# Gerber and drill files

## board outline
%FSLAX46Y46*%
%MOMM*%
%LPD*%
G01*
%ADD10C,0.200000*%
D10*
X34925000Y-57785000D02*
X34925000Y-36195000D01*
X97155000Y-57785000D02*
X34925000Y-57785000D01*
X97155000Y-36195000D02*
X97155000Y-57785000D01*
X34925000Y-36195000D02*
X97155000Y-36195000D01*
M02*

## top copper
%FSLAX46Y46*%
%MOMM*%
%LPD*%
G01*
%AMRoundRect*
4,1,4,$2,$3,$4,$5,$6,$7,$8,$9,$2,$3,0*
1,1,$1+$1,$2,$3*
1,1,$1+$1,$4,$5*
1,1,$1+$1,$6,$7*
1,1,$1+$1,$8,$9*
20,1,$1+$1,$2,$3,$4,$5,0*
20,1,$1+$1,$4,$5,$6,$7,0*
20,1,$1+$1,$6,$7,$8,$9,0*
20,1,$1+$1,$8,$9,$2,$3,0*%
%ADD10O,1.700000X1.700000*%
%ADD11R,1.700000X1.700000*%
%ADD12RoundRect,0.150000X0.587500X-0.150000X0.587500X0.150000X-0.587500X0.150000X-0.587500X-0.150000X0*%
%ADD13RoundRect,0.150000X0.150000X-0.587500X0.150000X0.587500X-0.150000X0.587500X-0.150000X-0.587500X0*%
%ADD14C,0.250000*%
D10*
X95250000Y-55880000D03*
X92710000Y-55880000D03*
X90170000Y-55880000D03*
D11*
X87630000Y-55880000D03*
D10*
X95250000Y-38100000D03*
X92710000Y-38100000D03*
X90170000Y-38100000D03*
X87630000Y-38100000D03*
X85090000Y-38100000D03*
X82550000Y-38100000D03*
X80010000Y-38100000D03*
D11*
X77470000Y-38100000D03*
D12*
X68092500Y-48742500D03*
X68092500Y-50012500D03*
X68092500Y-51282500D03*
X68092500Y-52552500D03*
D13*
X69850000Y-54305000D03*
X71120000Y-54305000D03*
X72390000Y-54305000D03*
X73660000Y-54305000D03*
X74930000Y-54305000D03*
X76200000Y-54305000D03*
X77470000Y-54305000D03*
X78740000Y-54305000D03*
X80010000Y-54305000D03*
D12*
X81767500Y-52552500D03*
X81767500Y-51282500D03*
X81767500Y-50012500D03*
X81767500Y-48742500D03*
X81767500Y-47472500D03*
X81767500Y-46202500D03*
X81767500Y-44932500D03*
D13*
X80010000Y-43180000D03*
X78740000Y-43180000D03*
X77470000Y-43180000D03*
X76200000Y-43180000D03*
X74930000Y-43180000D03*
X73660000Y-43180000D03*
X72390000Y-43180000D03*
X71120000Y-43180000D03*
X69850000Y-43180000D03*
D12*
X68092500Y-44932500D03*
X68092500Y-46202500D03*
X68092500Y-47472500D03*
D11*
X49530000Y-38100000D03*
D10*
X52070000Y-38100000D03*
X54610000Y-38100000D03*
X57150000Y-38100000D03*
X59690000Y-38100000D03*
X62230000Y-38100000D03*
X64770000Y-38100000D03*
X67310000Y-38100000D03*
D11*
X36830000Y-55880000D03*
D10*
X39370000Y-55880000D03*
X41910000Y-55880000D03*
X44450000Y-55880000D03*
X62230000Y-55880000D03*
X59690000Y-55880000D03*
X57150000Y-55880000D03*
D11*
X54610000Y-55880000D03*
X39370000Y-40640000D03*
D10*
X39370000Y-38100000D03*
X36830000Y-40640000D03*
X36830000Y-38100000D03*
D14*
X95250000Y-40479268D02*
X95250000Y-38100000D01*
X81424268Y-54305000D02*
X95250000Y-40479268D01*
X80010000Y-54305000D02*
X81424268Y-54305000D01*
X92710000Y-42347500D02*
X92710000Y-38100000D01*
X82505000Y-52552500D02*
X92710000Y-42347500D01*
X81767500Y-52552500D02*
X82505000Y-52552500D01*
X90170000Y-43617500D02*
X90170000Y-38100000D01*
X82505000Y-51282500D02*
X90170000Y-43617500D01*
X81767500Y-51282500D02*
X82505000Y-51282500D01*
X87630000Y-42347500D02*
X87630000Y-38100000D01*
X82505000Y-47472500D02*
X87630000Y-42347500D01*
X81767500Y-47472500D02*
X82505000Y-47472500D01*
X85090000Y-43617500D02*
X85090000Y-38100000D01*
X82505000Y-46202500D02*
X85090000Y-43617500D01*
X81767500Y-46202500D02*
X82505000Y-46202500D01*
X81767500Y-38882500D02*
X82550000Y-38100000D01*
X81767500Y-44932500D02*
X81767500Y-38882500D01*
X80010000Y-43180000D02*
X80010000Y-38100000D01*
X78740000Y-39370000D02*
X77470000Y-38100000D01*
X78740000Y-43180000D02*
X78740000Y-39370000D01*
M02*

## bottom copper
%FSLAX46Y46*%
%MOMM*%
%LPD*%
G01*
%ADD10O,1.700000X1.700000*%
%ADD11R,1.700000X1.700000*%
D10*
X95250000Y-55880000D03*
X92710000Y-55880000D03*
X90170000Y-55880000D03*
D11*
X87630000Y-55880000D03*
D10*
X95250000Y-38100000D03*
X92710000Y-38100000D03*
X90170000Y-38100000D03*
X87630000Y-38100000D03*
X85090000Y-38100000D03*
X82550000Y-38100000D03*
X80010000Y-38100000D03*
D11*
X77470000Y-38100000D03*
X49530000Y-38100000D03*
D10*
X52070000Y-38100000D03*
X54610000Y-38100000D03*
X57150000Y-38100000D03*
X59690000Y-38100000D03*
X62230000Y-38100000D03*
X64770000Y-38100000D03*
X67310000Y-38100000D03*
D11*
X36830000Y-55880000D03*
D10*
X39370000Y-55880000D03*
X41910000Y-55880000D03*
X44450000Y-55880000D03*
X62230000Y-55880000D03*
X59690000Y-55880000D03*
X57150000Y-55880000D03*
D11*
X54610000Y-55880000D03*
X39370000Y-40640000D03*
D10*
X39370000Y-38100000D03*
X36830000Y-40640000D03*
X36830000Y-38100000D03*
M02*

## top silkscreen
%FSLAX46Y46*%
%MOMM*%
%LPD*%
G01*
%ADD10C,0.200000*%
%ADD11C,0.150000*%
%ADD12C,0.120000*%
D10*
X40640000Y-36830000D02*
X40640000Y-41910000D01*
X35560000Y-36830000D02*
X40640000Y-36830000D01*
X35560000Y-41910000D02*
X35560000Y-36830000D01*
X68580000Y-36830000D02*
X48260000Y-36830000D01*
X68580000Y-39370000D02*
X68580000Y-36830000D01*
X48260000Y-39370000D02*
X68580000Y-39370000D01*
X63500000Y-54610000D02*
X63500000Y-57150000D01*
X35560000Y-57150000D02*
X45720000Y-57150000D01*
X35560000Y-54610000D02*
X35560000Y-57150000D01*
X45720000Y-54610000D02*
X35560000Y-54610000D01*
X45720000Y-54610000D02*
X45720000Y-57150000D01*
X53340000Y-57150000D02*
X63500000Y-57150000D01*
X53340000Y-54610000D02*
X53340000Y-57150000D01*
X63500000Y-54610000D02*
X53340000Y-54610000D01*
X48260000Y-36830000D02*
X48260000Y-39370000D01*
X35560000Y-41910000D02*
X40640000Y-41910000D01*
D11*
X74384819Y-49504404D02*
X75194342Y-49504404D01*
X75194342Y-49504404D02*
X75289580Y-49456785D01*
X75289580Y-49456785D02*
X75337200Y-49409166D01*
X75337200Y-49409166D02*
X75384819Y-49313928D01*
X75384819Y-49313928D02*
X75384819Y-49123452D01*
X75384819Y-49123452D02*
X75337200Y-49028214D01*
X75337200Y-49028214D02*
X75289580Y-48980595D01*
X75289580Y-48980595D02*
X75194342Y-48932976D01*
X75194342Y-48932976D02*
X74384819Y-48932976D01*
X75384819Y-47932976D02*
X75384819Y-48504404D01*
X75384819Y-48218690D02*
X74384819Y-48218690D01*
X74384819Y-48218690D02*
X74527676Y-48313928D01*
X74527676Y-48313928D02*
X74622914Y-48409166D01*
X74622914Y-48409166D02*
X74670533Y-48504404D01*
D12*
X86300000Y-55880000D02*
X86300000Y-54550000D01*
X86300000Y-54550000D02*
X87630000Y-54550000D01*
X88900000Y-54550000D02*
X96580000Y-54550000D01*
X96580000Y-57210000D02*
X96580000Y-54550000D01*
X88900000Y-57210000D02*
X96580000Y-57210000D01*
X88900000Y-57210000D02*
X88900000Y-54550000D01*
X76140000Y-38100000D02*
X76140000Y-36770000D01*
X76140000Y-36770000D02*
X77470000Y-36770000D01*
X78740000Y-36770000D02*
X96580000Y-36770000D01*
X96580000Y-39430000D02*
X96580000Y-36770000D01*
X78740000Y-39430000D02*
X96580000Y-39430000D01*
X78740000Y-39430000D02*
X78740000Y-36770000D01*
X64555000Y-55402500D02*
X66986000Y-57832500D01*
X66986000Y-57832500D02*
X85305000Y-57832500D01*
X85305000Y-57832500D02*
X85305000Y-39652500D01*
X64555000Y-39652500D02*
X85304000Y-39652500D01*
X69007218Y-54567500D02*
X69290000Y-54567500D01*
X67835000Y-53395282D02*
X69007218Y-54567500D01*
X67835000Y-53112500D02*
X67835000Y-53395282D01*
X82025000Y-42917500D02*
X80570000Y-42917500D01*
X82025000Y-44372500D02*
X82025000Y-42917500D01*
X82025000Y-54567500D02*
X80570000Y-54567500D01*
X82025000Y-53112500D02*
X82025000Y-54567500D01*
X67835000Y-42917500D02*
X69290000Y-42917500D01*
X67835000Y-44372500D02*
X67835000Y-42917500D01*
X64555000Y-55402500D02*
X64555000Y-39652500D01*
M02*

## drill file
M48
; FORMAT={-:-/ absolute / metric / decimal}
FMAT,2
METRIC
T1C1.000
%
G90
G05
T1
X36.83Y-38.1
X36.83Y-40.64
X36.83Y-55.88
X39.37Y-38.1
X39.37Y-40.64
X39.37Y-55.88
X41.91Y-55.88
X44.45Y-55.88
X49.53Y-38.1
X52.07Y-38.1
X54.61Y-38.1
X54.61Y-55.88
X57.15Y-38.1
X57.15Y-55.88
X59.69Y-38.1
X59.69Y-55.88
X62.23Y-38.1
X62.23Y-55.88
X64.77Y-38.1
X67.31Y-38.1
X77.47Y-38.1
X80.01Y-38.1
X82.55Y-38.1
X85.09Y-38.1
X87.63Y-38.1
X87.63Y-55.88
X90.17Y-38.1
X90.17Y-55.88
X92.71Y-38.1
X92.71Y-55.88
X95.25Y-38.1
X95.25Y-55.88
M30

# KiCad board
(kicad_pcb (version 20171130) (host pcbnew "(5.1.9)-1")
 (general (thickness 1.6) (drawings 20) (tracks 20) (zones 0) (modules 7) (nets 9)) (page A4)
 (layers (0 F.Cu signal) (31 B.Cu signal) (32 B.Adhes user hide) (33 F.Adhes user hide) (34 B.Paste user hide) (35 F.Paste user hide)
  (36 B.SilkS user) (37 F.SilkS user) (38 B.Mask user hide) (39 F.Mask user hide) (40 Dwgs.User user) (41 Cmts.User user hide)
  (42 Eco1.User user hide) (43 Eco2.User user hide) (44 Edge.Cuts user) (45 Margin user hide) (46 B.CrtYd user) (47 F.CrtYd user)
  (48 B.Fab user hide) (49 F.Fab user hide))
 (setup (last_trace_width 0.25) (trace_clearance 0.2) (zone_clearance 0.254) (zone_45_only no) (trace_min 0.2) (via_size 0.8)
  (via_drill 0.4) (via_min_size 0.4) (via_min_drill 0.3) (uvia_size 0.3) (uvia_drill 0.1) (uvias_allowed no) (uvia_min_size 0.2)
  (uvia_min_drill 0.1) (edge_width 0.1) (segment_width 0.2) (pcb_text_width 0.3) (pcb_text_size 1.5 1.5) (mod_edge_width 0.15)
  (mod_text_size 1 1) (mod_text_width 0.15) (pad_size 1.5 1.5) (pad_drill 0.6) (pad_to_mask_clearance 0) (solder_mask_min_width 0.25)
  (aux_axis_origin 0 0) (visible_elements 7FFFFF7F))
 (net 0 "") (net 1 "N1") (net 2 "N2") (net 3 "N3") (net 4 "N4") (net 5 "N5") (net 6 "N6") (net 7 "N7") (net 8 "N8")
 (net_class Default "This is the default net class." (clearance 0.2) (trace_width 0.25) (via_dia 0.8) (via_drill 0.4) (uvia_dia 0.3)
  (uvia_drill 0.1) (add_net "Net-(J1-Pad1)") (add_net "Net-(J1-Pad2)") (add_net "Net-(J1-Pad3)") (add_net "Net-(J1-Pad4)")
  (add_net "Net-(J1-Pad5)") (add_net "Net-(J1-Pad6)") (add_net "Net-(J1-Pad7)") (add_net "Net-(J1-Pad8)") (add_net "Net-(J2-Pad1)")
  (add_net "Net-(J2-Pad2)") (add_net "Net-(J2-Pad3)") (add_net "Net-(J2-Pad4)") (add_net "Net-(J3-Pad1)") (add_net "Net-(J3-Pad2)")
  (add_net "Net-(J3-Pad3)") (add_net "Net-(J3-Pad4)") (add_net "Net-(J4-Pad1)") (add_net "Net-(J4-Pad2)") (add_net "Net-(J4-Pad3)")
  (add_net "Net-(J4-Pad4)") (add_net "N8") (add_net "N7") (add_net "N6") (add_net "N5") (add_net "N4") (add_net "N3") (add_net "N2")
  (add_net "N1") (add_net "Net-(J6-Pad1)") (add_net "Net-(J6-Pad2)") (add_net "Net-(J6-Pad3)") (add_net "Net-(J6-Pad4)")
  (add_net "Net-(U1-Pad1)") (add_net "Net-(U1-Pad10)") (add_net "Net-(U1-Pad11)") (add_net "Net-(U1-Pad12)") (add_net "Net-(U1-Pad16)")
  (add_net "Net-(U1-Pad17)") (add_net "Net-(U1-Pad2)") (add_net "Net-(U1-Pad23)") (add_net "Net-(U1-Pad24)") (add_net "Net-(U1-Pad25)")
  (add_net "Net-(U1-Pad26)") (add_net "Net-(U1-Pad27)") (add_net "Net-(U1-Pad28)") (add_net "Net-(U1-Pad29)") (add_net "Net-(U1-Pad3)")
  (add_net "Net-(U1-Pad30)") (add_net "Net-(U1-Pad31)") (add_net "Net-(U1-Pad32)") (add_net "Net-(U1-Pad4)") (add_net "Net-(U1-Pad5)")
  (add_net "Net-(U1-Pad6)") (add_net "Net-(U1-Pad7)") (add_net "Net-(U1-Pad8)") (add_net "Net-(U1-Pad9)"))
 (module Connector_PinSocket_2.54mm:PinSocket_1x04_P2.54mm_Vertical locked (layer F.Cu) (at 87.63 55.88 90)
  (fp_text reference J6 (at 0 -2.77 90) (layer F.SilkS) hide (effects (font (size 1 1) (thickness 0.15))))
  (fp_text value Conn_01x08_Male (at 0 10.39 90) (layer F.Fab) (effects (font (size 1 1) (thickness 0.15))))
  (fp_line (start 0 -1.33) (end 1.33 -1.33) (layer F.SilkS) (width 0.12))
  (fp_line (start 1.33 -1.33) (end 1.33 0) (layer F.SilkS) (width 0.12))
  (fp_line (start 1.33 1.27) (end 1.33 8.95) (layer F.SilkS) (width 0.12))
  (fp_line (start -1.33 8.95) (end 1.33 8.95) (layer F.SilkS) (width 0.12))
  (fp_line (start -1.33 1.27) (end -1.33 8.95) (layer F.SilkS) (width 0.12))
  (fp_line (start -1.33 1.27) (end 1.33 1.27) (layer F.SilkS) (width 0.12))
  (pad 4 thru_hole oval (at 0 7.62 90) (size 1.7 1.7) (drill 1) (layers *.Cu *.Mask))
  (pad 3 thru_hole oval (at 0 5.08 90) (size 1.7 1.7) (drill 1) (layers *.Cu *.Mask))
  (pad 2 thru_hole oval (at 0 2.54 90) (size 1.7 1.7) (drill 1) (layers *.Cu *.Mask))
  (pad 1 thru_hole rect (at 0 0 90) (size 1.7 1.7) (drill 1) (layers *.Cu *.Mask)))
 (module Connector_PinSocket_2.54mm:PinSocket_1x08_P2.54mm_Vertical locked (layer F.Cu) (at 77.47 38.1 90)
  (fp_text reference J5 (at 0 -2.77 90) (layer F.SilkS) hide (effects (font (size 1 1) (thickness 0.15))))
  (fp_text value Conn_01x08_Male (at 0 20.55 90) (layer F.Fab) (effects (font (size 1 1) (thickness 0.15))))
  (fp_line (start 0 -1.33) (end 1.33 -1.33) (layer F.SilkS) (width 0.12))
  (fp_line (start 1.33 -1.33) (end 1.33 0) (layer F.SilkS) (width 0.12))
  (fp_line (start 1.33 1.27) (end 1.33 19.11) (layer F.SilkS) (width 0.12))
  (fp_line (start -1.33 19.11) (end 1.33 19.11) (layer F.SilkS) (width 0.12))
  (fp_line (start -1.33 1.27) (end -1.33 19.11) (layer F.SilkS) (width 0.12))
  (fp_line (start -1.33 1.27) (end 1.33 1.27) (layer F.SilkS) (width 0.12))
  (pad 8 thru_hole oval (at 0 17.78 90) (size 1.7 1.7) (drill 1) (layers *.Cu *.Mask) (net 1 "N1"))
  (pad 7 thru_hole oval (at 0 15.24 90) (size 1.7 1.7) (drill 1) (layers *.Cu *.Mask) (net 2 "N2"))
  (pad 6 thru_hole oval (at 0 12.7 90) (size 1.7 1.7) (drill 1) (layers *.Cu *.Mask) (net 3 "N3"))
  (pad 5 thru_hole oval (at 0 10.16 90) (size 1.7 1.7) (drill 1) (layers *.Cu *.Mask) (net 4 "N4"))
  (pad 4 thru_hole oval (at 0 7.62 90) (size 1.7 1.7) (drill 1) (layers *.Cu *.Mask) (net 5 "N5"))
  (pad 3 thru_hole oval (at 0 5.08 90) (size 1.7 1.7) (drill 1) (layers *.Cu *.Mask) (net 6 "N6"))
  (pad 2 thru_hole oval (at 0 2.54 90) (size 1.7 1.7) (drill 1) (layers *.Cu *.Mask) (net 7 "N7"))
  (pad 1 thru_hole rect (at 0 0 90) (size 1.7 1.7) (drill 1) (layers *.Cu *.Mask) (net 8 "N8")))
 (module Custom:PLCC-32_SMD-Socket (layer F.Cu) (at 74.93 48.7425 90)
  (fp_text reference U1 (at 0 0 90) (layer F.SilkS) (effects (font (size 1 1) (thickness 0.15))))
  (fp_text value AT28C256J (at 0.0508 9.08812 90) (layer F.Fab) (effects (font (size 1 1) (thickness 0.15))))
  (fp_line (start -6.66 -10.375) (end -9.09 -7.944) (layer F.SilkS) (width 0.12))
  (fp_line (start -9.09 -7.944) (end -9.09 10.375) (layer F.SilkS) (width 0.12))
  (fp_line (start -9.09 10.375) (end 9.09 10.375) (layer F.SilkS) (width 0.12))
  (fp_line (start 9.09 -10.375) (end 9.09 10.374) (layer F.SilkS) (width 0.12))
  (fp_line (start -5.825 -5.922782) (end -5.825 -5.64) (layer F.SilkS) (width 0.12))
  (fp_line (start -4.652782 -7.095) (end -5.825 -5.922782) (layer F.SilkS) (width 0.12))
  (fp_line (start -4.37 -7.095) (end -4.652782 -7.095) (layer F.SilkS) (width 0.12))
  (fp_line (start 5.825 7.095) (end 5.825 5.64) (layer F.SilkS) (width 0.12))
  (fp_line (start 4.37 7.095) (end 5.825 7.095) (layer F.SilkS) (width 0.12))
  (fp_line (start -5.825 7.095) (end -5.825 5.64) (layer F.SilkS) (width 0.12))
  (fp_line (start -4.37 7.095) (end -5.825 7.095) (layer F.SilkS) (width 0.12))
  (fp_line (start 5.825 -7.095) (end 5.825 -5.64) (layer F.SilkS) (width 0.12))
  (fp_line (start 4.37 -7.095) (end 5.825 -7.095) (layer F.SilkS) (width 0.12))
  (fp_line (start -6.66 -10.375) (end 9.09 -10.375) (layer F.SilkS) (width 0.12))
  (pad 1 smd roundrect (at 0 -6.8375 90) (size 0.6 1.475) (layers F.Cu F.Paste F.Mask) (roundrect_rratio 0.25))
  (pad 2 smd roundrect (at -1.27 -6.8375 90) (size 0.6 1.475) (layers F.Cu F.Paste F.Mask) (roundrect_rratio 0.25))
  (pad 3 smd roundrect (at -2.54 -6.8375 90) (size 0.6 1.475) (layers F.Cu F.Paste F.Mask) (roundrect_rratio 0.25))
  (pad 4 smd roundrect (at -3.81 -6.8375 90) (size 0.6 1.475) (layers F.Cu F.Paste F.Mask) (roundrect_rratio 0.25))
  (pad 5 smd roundrect (at -5.5625 -5.08 90) (size 1.475 0.6) (layers F.Cu F.Paste F.Mask) (roundrect_rratio 0.25))
  (pad 6 smd roundrect (at -5.5625 -3.81 90) (size 1.475 0.6) (layers F.Cu F.Paste F.Mask) (roundrect_rratio 0.25))
  (pad 7 smd roundrect (at -5.5625 -2.54 90) (size 1.475 0.6) (layers F.Cu F.Paste F.Mask) (roundrect_rratio 0.25))
  (pad 8 smd roundrect (at -5.5625 -1.27 90) (size 1.475 0.6) (layers F.Cu F.Paste F.Mask) (roundrect_rratio 0.25))
  (pad 9 smd roundrect (at -5.5625 0 90) (size 1.475 0.6) (layers F.Cu F.Paste F.Mask) (roundrect_rratio 0.25))
  (pad 10 smd roundrect (at -5.5625 1.27 90) (size 1.475 0.6) (layers F.Cu F.Paste F.Mask) (roundrect_rratio 0.25))
  (pad 11 smd roundrect (at -5.5625 2.54 90) (size 1.475 0.6) (layers F.Cu F.Paste F.Mask) (roundrect_rratio 0.25))
  (pad 12 smd roundrect (at -5.5625 3.81 90) (size 1.475 0.6) (layers F.Cu F.Paste F.Mask) (roundrect_rratio 0.25))
  (pad 13 smd roundrect (at -5.5625 5.08 90) (size 1.475 0.6) (layers F.Cu F.Paste F.Mask) (roundrect_rratio 0.25) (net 1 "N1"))
  (pad 14 smd roundrect (at -3.81 6.8375 90) (size 0.6 1.475) (layers F.Cu F.Paste F.Mask) (roundrect_rratio 0.25) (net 2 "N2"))
  (pad 15 smd roundrect (at -2.54 6.8375 90) (size 0.6 1.475) (layers F.Cu F.Paste F.Mask) (roundrect_rratio 0.25) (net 3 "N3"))
  (pad 16 smd roundrect (at -1.27 6.8375 90) (size 0.6 1.475) (layers F.Cu F.Paste F.Mask) (roundrect_rratio 0.25))
  (pad 17 smd roundrect (at 0 6.8375 90) (size 0.6 1.475) (layers F.Cu F.Paste F.Mask) (roundrect_rratio 0.25))
  (pad 18 smd roundrect (at 1.27 6.8375 90) (size 0.6 1.475) (layers F.Cu F.Paste F.Mask) (roundrect_rratio 0.25) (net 4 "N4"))
  (pad 19 smd roundrect (at 2.54 6.8375 90) (size 0.6 1.475) (layers F.Cu F.Paste F.Mask) (roundrect_rratio 0.25) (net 5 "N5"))
  (pad 20 smd roundrect (at 3.81 6.8375 90) (size 0.6 1.475) (layers F.Cu F.Paste F.Mask) (roundrect_rratio 0.25) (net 6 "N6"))
  (pad 21 smd roundrect (at 5.5625 5.08 90) (size 1.475 0.6) (layers F.Cu F.Paste F.Mask) (roundrect_rratio 0.25) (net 7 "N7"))
  (pad 22 smd roundrect (at 5.5625 3.81 90) (size 1.475 0.6) (layers F.Cu F.Paste F.Mask) (roundrect_rratio 0.25) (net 8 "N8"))
  (pad 23 smd roundrect (at 5.5625 2.54 90) (size 1.475 0.6) (layers F.Cu F.Paste F.Mask) (roundrect_rratio 0.25))
  (pad 24 smd roundrect (at 5.5625 1.27 90) (size 1.475 0.6) (layers F.Cu F.Paste F.Mask) (roundrect_rratio 0.25))
  (pad 25 smd roundrect (at 5.5625 0 90) (size 1.475 0.6) (layers F.Cu F.Paste F.Mask) (roundrect_rratio 0.25))
  (pad 26 smd roundrect (at 5.5625 -1.27 90) (size 1.475 0.6) (layers F.Cu F.Paste F.Mask) (roundrect_rratio 0.25))
  (pad 27 smd roundrect (at 5.5625 -2.54 90) (size 1.475 0.6) (layers F.Cu F.Paste F.Mask) (roundrect_rratio 0.25))
  (pad 28 smd roundrect (at 5.5625 -3.81 90) (size 1.475 0.6) (layers F.Cu F.Paste F.Mask) (roundrect_rratio 0.25))
  (pad 29 smd roundrect (at 5.5625 -5.08 90) (size 1.475 0.6) (layers F.Cu F.Paste F.Mask) (roundrect_rratio 0.25))
  (pad 30 smd roundrect (at 3.81 -6.8375 90) (size 0.6 1.475) (layers F.Cu F.Paste F.Mask) (roundrect_rratio 0.25))
  (pad 31 smd roundrect (at 2.54 -6.8375 90) (size 0.6 1.475) (layers F.Cu F.Paste F.Mask) (roundrect_rratio 0.25))
  (pad 32 smd roundrect (at 1.27 -6.8375 90) (size 0.6 1.475) (layers F.Cu F.Paste F.Mask) (roundrect_rratio 0.25)))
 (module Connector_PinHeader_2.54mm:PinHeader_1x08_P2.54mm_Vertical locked (layer B.Cu) (at 49.53 38.1 270)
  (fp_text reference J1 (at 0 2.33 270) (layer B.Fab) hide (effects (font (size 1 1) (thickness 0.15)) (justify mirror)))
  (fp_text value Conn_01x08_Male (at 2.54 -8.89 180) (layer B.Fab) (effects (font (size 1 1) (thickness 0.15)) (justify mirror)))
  (pad 1 thru_hole rect (at 0 0 270) (size 1.7 1.7) (drill 1) (layers *.Cu *.Mask))
  (pad 2 thru_hole oval (at 0 -2.54 270) (size 1.7 1.7) (drill 1) (layers *.Cu *.Mask))
  (pad 3 thru_hole oval (at 0 -5.08 270) (size 1.7 1.7) (drill 1) (layers *.Cu *.Mask))
  (pad 4 thru_hole oval (at 0 -7.62 270) (size 1.7 1.7) (drill 1) (layers *.Cu *.Mask))
  (pad 5 thru_hole oval (at 0 -10.16 270) (size 1.7 1.7) (drill 1) (layers *.Cu *.Mask))
  (pad 6 thru_hole oval (at 0 -12.7 270) (size 1.7 1.7) (drill 1) (layers *.Cu *.Mask))
  (pad 7 thru_hole oval (at 0 -15.24 270) (size 1.7 1.7) (drill 1) (layers *.Cu *.Mask))
  (pad 8 thru_hole oval (at 0 -17.78 270) (size 1.7 1.7) (drill 1) (layers *.Cu *.Mask)))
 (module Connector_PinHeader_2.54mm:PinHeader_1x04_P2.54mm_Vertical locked (layer B.Cu) (at 36.83 55.88 270)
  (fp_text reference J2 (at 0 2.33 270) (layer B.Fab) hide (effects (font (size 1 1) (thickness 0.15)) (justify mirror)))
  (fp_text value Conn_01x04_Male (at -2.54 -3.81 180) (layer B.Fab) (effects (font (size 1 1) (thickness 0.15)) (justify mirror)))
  (pad 1 thru_hole rect (at 0 0 270) (size 1.7 1.7) (drill 1) (layers *.Cu *.Mask))
  (pad 2 thru_hole oval (at 0 -2.54 270) (size 1.7 1.7) (drill 1) (layers *.Cu *.Mask))
  (pad 3 thru_hole oval (at 0 -5.08 270) (size 1.7 1.7) (drill 1) (layers *.Cu *.Mask))
  (pad 4 thru_hole oval (at 0 -7.62 270) (size 1.7 1.7) (drill 1) (layers *.Cu *.Mask)))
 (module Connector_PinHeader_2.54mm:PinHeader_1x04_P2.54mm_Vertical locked (layer B.Cu) (at 54.61 55.88 270)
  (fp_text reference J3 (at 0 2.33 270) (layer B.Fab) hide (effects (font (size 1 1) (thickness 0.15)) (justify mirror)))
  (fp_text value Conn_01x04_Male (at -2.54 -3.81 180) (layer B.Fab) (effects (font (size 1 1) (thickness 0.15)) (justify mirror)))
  (pad 4 thru_hole oval (at 0 -7.62 270) (size 1.7 1.7) (drill 1) (layers *.Cu *.Mask))
  (pad 3 thru_hole oval (at 0 -5.08 270) (size 1.7 1.7) (drill 1) (layers *.Cu *.Mask))
  (pad 2 thru_hole oval (at 0 -2.54 270) (size 1.7 1.7) (drill 1) (layers *.Cu *.Mask))
  (pad 1 thru_hole rect (at 0 0 270) (size 1.7 1.7) (drill 1) (layers *.Cu *.Mask)))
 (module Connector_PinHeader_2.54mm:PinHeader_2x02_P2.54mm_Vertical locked (layer B.Cu) (at 39.37 40.64 90)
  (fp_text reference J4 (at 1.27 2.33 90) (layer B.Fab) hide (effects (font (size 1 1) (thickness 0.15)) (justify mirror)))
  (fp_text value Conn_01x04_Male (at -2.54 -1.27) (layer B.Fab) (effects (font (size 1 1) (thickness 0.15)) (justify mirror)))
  (pad 1 thru_hole rect (at 0 0 90) (size 1.7 1.7) (drill 1) (layers *.Cu *.Mask))
  (pad 2 thru_hole oval (at 2.54 0 90) (size 1.7 1.7) (drill 1) (layers *.Cu *.Mask))
  (pad 3 thru_hole oval (at 0 -2.54 90) (size 1.7 1.7) (drill 1) (layers *.Cu *.Mask))
  (pad 4 thru_hole oval (at 2.54 -2.54 90) (size 1.7 1.7) (drill 1) (layers *.Cu *.Mask)))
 (gr_line (start 40.64 36.83) (end 40.64 41.91) (layer F.SilkS) (width 0.2))
 (gr_line (start 35.56 36.83) (end 40.64 36.83) (layer F.SilkS) (width 0.2))
 (gr_line (start 35.56 41.91) (end 35.56 36.83) (layer F.SilkS) (width 0.2))
 (gr_line (start 68.58 36.83) (end 48.26 36.83) (layer F.SilkS) (width 0.2))
 (gr_line (start 68.58 39.37) (end 68.58 36.83) (layer F.SilkS) (width 0.2))
 (gr_line (start 48.26 39.37) (end 68.58 39.37) (layer F.SilkS) (width 0.2))
 (gr_line (start 63.5 54.61) (end 63.5 57.15) (layer F.SilkS) (width 0.2))
 (gr_line (start 35.56 57.15) (end 45.72 57.15) (layer F.SilkS) (width 0.2))
 (gr_line (start 35.56 54.61) (end 35.56 57.15) (layer F.SilkS) (width 0.2))
 (gr_line (start 45.72 54.61) (end 35.56 54.61) (layer F.SilkS) (width 0.2))
 (gr_line (start 45.72 54.61) (end 45.72 57.15) (layer F.SilkS) (width 0.2))
 (gr_line (start 53.34 57.15) (end 63.5 57.15) (layer F.SilkS) (width 0.2))
 (gr_line (start 53.34 54.61) (end 53.34 57.15) (layer F.SilkS) (width 0.2))
 (gr_line (start 63.5 54.61) (end 53.34 54.61) (layer F.SilkS) (width 0.2))
 (gr_line (start 48.26 36.83) (end 48.26 39.37) (layer F.SilkS) (width 0.2))
 (gr_line (start 35.56 41.91) (end 40.64 41.91) (layer F.SilkS) (width 0.2))
 (gr_line (start 34.925 57.785) (end 34.925 36.195) (layer Edge.Cuts) (width 0.2))
 (gr_line (start 97.155 57.785) (end 34.925 57.785) (layer Edge.Cuts) (width 0.2))
 (gr_line (start 97.155 36.195) (end 97.155 57.785) (layer Edge.Cuts) (width 0.2))
 (gr_line (start 34.925 36.195) (end 97.155 36.195) (layer Edge.Cuts) (width 0.2))
 (segment (start 95.25 40.479268) (end 95.25 38.1) (width 0.25) (layer F.Cu) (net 1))
 (segment (start 81.424268 54.305) (end 95.25 40.479268) (width 0.25) (layer F.Cu) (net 1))
 (segment (start 80.01 54.305) (end 81.424268 54.305) (width 0.25) (layer F.Cu) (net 1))
 (segment (start 92.71 42.3475) (end 92.71 38.1) (width 0.25) (layer F.Cu) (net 2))
 (segment (start 82.505 52.5525) (end 92.71 42.3475) (width 0.25) (layer F.Cu) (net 2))
 (segment (start 81.7675 52.5525) (end 82.505 52.5525) (width 0.25) (layer F.Cu) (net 2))
 (segment (start 90.17 43.6175) (end 90.17 38.1) (width 0.25) (layer F.Cu) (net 3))
 (segment (start 82.505 51.2825) (end 90.17 43.6175) (width 0.25) (layer F.Cu) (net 3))
 (segment (start 81.7675 51.2825) (end 82.505 51.2825) (width 0.25) (layer F.Cu) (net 3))
 (segment (start 87.63 42.3475) (end 87.63 38.1) (width 0.25) (layer F.Cu) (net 4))
 (segment (start 82.505 47.4725) (end 87.63 42.3475) (width 0.25) (layer F.Cu) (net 4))
 (segment (start 81.7675 47.4725) (end 82.505 47.4725) (width 0.25) (layer F.Cu) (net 4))
 (segment (start 85.09 43.6175) (end 85.09 38.1) (width 0.25) (layer F.Cu) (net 5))
 (segment (start 82.505 46.2025) (end 85.09 43.6175) (width 0.25) (layer F.Cu) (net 5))
 (segment (start 81.7675 46.2025) (end 82.505 46.2025) (width 0.25) (layer F.Cu) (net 5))
 (segment (start 81.7675 38.8825) (end 82.55 38.1) (width 0.25) (layer F.Cu) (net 6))
 (segment (start 81.7675 44.9325) (end 81.7675 38.8825) (width 0.25) (layer F.Cu) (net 6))
 (segment (start 80.01 43.18) (end 80.01 38.1) (width 0.25) (layer F.Cu) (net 7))
 (segment (start 78.74 39.37) (end 77.47 38.1) (width 0.25) (layer F.Cu) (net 8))
 (segment (start 78.74 43.18) (end 78.74 39.37) (width 0.25) (layer F.Cu) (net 8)))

